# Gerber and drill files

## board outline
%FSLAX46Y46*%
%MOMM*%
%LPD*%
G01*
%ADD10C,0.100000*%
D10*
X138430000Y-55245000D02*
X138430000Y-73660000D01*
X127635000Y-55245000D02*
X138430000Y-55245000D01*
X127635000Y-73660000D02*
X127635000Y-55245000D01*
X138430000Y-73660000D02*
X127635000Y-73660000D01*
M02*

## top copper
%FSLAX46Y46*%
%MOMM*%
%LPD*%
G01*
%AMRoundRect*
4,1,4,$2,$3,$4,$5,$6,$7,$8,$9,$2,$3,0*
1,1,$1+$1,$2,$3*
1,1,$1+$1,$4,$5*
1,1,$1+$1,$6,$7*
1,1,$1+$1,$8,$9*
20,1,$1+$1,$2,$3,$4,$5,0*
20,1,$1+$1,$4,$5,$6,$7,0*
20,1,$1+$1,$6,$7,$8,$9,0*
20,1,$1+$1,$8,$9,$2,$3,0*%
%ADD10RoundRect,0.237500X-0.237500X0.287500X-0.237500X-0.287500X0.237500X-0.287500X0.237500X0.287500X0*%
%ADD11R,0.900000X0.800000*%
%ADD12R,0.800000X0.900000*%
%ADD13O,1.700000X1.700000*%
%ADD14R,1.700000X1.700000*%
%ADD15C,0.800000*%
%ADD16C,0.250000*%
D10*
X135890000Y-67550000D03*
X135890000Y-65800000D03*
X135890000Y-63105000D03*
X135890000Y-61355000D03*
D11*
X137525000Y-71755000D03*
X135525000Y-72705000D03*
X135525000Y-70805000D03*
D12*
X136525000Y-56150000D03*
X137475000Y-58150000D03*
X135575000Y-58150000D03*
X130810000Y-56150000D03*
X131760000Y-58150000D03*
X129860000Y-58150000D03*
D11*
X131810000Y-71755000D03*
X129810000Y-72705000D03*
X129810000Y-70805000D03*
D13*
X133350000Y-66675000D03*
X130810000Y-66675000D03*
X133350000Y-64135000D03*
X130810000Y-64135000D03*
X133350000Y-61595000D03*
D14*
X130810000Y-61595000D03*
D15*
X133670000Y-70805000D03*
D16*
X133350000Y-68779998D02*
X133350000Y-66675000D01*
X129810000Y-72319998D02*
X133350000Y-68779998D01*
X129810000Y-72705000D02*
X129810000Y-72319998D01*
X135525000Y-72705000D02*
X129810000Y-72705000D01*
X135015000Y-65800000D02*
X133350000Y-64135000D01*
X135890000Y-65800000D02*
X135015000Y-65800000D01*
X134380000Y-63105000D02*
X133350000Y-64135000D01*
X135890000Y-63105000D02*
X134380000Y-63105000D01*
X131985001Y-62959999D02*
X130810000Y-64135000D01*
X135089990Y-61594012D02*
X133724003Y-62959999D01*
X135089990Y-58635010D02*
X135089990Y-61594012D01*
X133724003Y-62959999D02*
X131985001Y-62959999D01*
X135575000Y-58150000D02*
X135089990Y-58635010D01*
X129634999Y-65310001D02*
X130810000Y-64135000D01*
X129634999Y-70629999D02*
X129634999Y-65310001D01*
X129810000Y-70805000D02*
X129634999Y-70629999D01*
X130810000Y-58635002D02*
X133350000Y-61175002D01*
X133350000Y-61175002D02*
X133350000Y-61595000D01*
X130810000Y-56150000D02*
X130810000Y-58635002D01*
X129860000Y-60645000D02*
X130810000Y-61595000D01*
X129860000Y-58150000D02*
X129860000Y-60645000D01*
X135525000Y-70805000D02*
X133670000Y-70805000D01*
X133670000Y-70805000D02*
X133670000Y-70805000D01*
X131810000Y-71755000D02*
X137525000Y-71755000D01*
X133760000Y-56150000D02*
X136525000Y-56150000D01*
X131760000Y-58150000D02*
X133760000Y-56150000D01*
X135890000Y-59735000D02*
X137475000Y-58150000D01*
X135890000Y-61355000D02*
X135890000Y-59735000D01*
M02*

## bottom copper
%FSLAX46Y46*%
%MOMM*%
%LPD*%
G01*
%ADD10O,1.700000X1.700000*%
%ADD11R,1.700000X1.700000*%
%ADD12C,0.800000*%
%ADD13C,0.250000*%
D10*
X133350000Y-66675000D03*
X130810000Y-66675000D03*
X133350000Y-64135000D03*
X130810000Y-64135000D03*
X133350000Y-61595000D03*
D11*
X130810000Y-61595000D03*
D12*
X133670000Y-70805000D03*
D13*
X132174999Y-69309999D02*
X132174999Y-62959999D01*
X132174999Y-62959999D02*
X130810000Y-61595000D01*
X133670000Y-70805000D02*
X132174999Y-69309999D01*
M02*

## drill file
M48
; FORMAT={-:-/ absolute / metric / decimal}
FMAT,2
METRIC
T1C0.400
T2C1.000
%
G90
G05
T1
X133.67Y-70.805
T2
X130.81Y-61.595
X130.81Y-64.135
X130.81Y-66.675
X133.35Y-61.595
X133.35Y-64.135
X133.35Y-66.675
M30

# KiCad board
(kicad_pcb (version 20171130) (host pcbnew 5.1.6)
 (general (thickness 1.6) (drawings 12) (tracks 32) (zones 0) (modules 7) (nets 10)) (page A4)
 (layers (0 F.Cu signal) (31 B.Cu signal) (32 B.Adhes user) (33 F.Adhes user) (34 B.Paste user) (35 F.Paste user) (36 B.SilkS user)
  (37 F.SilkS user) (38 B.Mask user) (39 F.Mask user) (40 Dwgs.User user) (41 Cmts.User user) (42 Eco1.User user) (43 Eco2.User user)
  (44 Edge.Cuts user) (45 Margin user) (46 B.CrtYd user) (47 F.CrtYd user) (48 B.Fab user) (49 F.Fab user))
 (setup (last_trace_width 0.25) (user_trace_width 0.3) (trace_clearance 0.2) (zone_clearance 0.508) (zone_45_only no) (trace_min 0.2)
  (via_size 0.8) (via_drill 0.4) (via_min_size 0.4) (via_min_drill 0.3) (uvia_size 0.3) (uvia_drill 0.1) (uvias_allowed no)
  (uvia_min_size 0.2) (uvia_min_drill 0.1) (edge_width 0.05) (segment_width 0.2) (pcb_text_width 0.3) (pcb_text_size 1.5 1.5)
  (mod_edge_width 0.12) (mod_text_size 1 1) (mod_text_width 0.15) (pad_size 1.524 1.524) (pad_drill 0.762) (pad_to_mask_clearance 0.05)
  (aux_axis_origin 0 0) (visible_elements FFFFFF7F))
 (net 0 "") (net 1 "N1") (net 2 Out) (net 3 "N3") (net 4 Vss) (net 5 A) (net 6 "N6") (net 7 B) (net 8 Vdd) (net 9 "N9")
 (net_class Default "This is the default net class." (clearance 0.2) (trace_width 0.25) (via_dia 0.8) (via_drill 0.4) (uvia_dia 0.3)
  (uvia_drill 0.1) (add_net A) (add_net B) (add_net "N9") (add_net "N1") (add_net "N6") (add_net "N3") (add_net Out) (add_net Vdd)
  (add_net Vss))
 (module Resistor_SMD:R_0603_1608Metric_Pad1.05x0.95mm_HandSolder (layer F.Cu) (at 135.89 66.675 270)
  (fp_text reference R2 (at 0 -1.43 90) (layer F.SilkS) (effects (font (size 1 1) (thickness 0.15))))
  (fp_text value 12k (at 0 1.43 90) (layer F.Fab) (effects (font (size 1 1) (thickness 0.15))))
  (pad 2 smd roundrect (at 0.875 0 270) (size 1.05 0.95) (layers F.Cu F.Paste F.Mask) (roundrect_rratio 0.25) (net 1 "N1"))
  (pad 1 smd roundrect (at -0.875 0 270) (size 1.05 0.95) (layers F.Cu F.Paste F.Mask) (roundrect_rratio 0.25) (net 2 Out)))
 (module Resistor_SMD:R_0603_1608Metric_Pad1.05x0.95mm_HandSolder (layer F.Cu) (at 135.89 62.23 270)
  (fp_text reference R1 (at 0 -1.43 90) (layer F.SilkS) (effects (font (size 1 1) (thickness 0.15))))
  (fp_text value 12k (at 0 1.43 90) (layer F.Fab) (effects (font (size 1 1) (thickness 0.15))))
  (pad 2 smd roundrect (at 0.875 0 270) (size 1.05 0.95) (layers F.Cu F.Paste F.Mask) (roundrect_rratio 0.25) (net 2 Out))
  (pad 1 smd roundrect (at -0.875 0 270) (size 1.05 0.95) (layers F.Cu F.Paste F.Mask) (roundrect_rratio 0.25) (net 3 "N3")))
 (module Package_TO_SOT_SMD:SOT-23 (layer F.Cu) (at 136.525 71.755)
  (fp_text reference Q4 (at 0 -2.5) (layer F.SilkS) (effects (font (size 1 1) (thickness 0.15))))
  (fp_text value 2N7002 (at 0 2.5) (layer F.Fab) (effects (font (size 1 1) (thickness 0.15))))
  (pad 3 smd rect (at 1 0) (size 0.9 0.8) (layers F.Cu F.Paste F.Mask) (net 1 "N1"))
  (pad 2 smd rect (at -1 0.95) (size 0.9 0.8) (layers F.Cu F.Paste F.Mask) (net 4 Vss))
  (pad 1 smd rect (at -1 -0.95) (size 0.9 0.8) (layers F.Cu F.Paste F.Mask) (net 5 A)))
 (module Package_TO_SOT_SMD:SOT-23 (layer F.Cu) (at 136.525 57.15 90)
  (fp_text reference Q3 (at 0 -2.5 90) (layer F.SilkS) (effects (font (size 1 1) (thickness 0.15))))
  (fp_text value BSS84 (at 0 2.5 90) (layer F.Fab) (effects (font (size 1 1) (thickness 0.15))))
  (pad 3 smd rect (at 1 0 90) (size 0.9 0.8) (layers F.Cu F.Paste F.Mask) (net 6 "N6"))
  (pad 2 smd rect (at -1 0.95 90) (size 0.9 0.8) (layers F.Cu F.Paste F.Mask) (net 3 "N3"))
  (pad 1 smd rect (at -1 -0.95 90) (size 0.9 0.8) (layers F.Cu F.Paste F.Mask) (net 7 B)))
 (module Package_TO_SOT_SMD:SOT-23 (layer F.Cu) (at 130.81 57.15 90)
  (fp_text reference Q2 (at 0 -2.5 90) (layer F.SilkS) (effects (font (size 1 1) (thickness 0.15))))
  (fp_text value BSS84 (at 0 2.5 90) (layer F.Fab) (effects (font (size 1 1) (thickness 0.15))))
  (pad 3 smd rect (at 1 0 90) (size 0.9 0.8) (layers F.Cu F.Paste F.Mask) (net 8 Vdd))
  (pad 2 smd rect (at -1 0.95 90) (size 0.9 0.8) (layers F.Cu F.Paste F.Mask) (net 6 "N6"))
  (pad 1 smd rect (at -1 -0.95 90) (size 0.9 0.8) (layers F.Cu F.Paste F.Mask) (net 5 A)))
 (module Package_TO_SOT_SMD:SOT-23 (layer F.Cu) (at 130.81 71.755)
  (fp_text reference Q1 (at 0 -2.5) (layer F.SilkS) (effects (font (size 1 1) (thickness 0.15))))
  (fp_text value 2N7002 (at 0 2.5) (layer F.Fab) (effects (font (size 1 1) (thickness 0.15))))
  (pad 3 smd rect (at 1 0) (size 0.9 0.8) (layers F.Cu F.Paste F.Mask) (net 1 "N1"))
  (pad 2 smd rect (at -1 0.95) (size 0.9 0.8) (layers F.Cu F.Paste F.Mask) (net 4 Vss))
  (pad 1 smd rect (at -1 -0.95) (size 0.9 0.8) (layers F.Cu F.Paste F.Mask) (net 7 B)))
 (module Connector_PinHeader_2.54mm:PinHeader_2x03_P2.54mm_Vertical (layer F.Cu) (at 130.81 61.595)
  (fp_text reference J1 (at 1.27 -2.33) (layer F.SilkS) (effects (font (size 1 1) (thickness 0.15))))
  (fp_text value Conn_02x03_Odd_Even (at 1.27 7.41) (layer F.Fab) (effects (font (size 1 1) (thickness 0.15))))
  (pad 6 thru_hole oval (at 2.54 5.08) (size 1.7 1.7) (drill 1) (layers *.Cu *.Mask) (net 4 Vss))
  (pad 5 thru_hole oval (at 0 5.08) (size 1.7 1.7) (drill 1) (layers *.Cu *.Mask) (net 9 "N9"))
  (pad 4 thru_hole oval (at 2.54 2.54) (size 1.7 1.7) (drill 1) (layers *.Cu *.Mask) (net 2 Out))
  (pad 3 thru_hole oval (at 0 2.54) (size 1.7 1.7) (drill 1) (layers *.Cu *.Mask) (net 7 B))
  (pad 2 thru_hole oval (at 2.54 0) (size 1.7 1.7) (drill 1) (layers *.Cu *.Mask) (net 8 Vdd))
  (pad 1 thru_hole rect (at 0 0) (size 1.7 1.7) (drill 1) (layers *.Cu *.Mask) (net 5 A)))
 (gr_line (start 138.43 55.245) (end 138.43 73.66) (layer Edge.Cuts) (width 0.1))
 (gr_line (start 127.635 55.245) (end 138.43 55.245) (layer Edge.Cuts) (width 0.1))
 (gr_line (start 127.635 73.66) (end 127.635 55.245) (layer Edge.Cuts) (width 0.1))
 (gr_line (start 138.43 73.66) (end 127.635 73.66) (layer Edge.Cuts) (width 0.1))
 (segment (start 133.35 68.779998) (end 133.35 66.675) (width 0.25) (layer F.Cu) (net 4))
 (segment (start 129.81 72.319998) (end 133.35 68.779998) (width 0.25) (layer F.Cu) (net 4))
 (segment (start 129.81 72.705) (end 129.81 72.319998) (width 0.25) (layer F.Cu) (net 4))
 (segment (start 135.525 72.705) (end 129.81 72.705) (width 0.25) (layer F.Cu) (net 4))
 (segment (start 135.015 65.8) (end 133.35 64.135) (width 0.25) (layer F.Cu) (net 2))
 (segment (start 135.89 65.8) (end 135.015 65.8) (width 0.25) (layer F.Cu) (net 2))
 (segment (start 134.38 63.105) (end 133.35 64.135) (width 0.25) (layer F.Cu) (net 2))
 (segment (start 135.89 63.105) (end 134.38 63.105) (width 0.25) (layer F.Cu) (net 2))
 (segment (start 131.985001 62.959999) (end 130.81 64.135) (width 0.25) (layer F.Cu) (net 7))
 (segment (start 135.08999 61.594012) (end 133.724003 62.959999) (width 0.25) (layer F.Cu) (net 7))
 (segment (start 135.08999 58.63501) (end 135.08999 61.594012) (width 0.25) (layer F.Cu) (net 7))
 (segment (start 133.724003 62.959999) (end 131.985001 62.959999) (width 0.25) (layer F.Cu) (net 7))
 (segment (start 135.575 58.15) (end 135.08999 58.63501) (width 0.25) (layer F.Cu) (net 7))
 (segment (start 129.634999 65.310001) (end 130.81 64.135) (width 0.25) (layer F.Cu) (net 7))
 (segment (start 129.634999 70.629999) (end 129.634999 65.310001) (width 0.25) (layer F.Cu) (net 7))
 (segment (start 129.81 70.805) (end 129.634999 70.629999) (width 0.25) (layer F.Cu) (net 7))
 (segment (start 130.81 58.635002) (end 133.35 61.175002) (width 0.25) (layer F.Cu) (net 8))
 (segment (start 133.35 61.175002) (end 133.35 61.595) (width 0.25) (layer F.Cu) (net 8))
 (segment (start 130.81 56.15) (end 130.81 58.635002) (width 0.25) (layer F.Cu) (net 8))
 (segment (start 129.86 60.645) (end 130.81 61.595) (width 0.25) (layer F.Cu) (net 5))
 (segment (start 129.86 58.15) (end 129.86 60.645) (width 0.25) (layer F.Cu) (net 5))
 (segment (start 135.525 70.805) (end 133.67 70.805) (width 0.25) (layer F.Cu) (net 5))
 (segment (start 133.67 70.805) (end 133.67 70.805) (width 0.25) (layer F.Cu) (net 5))
 (via (at 133.67 70.805) (size 0.8) (drill 0.4) (layers F.Cu B.Cu) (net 5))
 (segment (start 132.174999 69.309999) (end 132.174999 62.959999) (width 0.25) (layer B.Cu) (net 5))
 (segment (start 132.174999 62.959999) (end 130.81 61.595) (width 0.25) (layer B.Cu) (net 5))
 (segment (start 133.67 70.805) (end 132.174999 69.309999) (width 0.25) (layer B.Cu) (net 5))
 (segment (start 131.81 71.755) (end 137.525 71.755) (width 0.25) (layer F.Cu) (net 1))
 (segment (start 133.76 56.15) (end 136.525 56.15) (width 0.25) (layer F.Cu) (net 6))
 (segment (start 131.76 58.15) (end 133.76 56.15) (width 0.25) (layer F.Cu) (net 6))
 (segment (start 135.89 59.735) (end 137.475 58.15) (width 0.25) (layer F.Cu) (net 3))
 (segment (start 135.89 61.355) (end 135.89 59.735) (width 0.25) (layer F.Cu) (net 3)))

